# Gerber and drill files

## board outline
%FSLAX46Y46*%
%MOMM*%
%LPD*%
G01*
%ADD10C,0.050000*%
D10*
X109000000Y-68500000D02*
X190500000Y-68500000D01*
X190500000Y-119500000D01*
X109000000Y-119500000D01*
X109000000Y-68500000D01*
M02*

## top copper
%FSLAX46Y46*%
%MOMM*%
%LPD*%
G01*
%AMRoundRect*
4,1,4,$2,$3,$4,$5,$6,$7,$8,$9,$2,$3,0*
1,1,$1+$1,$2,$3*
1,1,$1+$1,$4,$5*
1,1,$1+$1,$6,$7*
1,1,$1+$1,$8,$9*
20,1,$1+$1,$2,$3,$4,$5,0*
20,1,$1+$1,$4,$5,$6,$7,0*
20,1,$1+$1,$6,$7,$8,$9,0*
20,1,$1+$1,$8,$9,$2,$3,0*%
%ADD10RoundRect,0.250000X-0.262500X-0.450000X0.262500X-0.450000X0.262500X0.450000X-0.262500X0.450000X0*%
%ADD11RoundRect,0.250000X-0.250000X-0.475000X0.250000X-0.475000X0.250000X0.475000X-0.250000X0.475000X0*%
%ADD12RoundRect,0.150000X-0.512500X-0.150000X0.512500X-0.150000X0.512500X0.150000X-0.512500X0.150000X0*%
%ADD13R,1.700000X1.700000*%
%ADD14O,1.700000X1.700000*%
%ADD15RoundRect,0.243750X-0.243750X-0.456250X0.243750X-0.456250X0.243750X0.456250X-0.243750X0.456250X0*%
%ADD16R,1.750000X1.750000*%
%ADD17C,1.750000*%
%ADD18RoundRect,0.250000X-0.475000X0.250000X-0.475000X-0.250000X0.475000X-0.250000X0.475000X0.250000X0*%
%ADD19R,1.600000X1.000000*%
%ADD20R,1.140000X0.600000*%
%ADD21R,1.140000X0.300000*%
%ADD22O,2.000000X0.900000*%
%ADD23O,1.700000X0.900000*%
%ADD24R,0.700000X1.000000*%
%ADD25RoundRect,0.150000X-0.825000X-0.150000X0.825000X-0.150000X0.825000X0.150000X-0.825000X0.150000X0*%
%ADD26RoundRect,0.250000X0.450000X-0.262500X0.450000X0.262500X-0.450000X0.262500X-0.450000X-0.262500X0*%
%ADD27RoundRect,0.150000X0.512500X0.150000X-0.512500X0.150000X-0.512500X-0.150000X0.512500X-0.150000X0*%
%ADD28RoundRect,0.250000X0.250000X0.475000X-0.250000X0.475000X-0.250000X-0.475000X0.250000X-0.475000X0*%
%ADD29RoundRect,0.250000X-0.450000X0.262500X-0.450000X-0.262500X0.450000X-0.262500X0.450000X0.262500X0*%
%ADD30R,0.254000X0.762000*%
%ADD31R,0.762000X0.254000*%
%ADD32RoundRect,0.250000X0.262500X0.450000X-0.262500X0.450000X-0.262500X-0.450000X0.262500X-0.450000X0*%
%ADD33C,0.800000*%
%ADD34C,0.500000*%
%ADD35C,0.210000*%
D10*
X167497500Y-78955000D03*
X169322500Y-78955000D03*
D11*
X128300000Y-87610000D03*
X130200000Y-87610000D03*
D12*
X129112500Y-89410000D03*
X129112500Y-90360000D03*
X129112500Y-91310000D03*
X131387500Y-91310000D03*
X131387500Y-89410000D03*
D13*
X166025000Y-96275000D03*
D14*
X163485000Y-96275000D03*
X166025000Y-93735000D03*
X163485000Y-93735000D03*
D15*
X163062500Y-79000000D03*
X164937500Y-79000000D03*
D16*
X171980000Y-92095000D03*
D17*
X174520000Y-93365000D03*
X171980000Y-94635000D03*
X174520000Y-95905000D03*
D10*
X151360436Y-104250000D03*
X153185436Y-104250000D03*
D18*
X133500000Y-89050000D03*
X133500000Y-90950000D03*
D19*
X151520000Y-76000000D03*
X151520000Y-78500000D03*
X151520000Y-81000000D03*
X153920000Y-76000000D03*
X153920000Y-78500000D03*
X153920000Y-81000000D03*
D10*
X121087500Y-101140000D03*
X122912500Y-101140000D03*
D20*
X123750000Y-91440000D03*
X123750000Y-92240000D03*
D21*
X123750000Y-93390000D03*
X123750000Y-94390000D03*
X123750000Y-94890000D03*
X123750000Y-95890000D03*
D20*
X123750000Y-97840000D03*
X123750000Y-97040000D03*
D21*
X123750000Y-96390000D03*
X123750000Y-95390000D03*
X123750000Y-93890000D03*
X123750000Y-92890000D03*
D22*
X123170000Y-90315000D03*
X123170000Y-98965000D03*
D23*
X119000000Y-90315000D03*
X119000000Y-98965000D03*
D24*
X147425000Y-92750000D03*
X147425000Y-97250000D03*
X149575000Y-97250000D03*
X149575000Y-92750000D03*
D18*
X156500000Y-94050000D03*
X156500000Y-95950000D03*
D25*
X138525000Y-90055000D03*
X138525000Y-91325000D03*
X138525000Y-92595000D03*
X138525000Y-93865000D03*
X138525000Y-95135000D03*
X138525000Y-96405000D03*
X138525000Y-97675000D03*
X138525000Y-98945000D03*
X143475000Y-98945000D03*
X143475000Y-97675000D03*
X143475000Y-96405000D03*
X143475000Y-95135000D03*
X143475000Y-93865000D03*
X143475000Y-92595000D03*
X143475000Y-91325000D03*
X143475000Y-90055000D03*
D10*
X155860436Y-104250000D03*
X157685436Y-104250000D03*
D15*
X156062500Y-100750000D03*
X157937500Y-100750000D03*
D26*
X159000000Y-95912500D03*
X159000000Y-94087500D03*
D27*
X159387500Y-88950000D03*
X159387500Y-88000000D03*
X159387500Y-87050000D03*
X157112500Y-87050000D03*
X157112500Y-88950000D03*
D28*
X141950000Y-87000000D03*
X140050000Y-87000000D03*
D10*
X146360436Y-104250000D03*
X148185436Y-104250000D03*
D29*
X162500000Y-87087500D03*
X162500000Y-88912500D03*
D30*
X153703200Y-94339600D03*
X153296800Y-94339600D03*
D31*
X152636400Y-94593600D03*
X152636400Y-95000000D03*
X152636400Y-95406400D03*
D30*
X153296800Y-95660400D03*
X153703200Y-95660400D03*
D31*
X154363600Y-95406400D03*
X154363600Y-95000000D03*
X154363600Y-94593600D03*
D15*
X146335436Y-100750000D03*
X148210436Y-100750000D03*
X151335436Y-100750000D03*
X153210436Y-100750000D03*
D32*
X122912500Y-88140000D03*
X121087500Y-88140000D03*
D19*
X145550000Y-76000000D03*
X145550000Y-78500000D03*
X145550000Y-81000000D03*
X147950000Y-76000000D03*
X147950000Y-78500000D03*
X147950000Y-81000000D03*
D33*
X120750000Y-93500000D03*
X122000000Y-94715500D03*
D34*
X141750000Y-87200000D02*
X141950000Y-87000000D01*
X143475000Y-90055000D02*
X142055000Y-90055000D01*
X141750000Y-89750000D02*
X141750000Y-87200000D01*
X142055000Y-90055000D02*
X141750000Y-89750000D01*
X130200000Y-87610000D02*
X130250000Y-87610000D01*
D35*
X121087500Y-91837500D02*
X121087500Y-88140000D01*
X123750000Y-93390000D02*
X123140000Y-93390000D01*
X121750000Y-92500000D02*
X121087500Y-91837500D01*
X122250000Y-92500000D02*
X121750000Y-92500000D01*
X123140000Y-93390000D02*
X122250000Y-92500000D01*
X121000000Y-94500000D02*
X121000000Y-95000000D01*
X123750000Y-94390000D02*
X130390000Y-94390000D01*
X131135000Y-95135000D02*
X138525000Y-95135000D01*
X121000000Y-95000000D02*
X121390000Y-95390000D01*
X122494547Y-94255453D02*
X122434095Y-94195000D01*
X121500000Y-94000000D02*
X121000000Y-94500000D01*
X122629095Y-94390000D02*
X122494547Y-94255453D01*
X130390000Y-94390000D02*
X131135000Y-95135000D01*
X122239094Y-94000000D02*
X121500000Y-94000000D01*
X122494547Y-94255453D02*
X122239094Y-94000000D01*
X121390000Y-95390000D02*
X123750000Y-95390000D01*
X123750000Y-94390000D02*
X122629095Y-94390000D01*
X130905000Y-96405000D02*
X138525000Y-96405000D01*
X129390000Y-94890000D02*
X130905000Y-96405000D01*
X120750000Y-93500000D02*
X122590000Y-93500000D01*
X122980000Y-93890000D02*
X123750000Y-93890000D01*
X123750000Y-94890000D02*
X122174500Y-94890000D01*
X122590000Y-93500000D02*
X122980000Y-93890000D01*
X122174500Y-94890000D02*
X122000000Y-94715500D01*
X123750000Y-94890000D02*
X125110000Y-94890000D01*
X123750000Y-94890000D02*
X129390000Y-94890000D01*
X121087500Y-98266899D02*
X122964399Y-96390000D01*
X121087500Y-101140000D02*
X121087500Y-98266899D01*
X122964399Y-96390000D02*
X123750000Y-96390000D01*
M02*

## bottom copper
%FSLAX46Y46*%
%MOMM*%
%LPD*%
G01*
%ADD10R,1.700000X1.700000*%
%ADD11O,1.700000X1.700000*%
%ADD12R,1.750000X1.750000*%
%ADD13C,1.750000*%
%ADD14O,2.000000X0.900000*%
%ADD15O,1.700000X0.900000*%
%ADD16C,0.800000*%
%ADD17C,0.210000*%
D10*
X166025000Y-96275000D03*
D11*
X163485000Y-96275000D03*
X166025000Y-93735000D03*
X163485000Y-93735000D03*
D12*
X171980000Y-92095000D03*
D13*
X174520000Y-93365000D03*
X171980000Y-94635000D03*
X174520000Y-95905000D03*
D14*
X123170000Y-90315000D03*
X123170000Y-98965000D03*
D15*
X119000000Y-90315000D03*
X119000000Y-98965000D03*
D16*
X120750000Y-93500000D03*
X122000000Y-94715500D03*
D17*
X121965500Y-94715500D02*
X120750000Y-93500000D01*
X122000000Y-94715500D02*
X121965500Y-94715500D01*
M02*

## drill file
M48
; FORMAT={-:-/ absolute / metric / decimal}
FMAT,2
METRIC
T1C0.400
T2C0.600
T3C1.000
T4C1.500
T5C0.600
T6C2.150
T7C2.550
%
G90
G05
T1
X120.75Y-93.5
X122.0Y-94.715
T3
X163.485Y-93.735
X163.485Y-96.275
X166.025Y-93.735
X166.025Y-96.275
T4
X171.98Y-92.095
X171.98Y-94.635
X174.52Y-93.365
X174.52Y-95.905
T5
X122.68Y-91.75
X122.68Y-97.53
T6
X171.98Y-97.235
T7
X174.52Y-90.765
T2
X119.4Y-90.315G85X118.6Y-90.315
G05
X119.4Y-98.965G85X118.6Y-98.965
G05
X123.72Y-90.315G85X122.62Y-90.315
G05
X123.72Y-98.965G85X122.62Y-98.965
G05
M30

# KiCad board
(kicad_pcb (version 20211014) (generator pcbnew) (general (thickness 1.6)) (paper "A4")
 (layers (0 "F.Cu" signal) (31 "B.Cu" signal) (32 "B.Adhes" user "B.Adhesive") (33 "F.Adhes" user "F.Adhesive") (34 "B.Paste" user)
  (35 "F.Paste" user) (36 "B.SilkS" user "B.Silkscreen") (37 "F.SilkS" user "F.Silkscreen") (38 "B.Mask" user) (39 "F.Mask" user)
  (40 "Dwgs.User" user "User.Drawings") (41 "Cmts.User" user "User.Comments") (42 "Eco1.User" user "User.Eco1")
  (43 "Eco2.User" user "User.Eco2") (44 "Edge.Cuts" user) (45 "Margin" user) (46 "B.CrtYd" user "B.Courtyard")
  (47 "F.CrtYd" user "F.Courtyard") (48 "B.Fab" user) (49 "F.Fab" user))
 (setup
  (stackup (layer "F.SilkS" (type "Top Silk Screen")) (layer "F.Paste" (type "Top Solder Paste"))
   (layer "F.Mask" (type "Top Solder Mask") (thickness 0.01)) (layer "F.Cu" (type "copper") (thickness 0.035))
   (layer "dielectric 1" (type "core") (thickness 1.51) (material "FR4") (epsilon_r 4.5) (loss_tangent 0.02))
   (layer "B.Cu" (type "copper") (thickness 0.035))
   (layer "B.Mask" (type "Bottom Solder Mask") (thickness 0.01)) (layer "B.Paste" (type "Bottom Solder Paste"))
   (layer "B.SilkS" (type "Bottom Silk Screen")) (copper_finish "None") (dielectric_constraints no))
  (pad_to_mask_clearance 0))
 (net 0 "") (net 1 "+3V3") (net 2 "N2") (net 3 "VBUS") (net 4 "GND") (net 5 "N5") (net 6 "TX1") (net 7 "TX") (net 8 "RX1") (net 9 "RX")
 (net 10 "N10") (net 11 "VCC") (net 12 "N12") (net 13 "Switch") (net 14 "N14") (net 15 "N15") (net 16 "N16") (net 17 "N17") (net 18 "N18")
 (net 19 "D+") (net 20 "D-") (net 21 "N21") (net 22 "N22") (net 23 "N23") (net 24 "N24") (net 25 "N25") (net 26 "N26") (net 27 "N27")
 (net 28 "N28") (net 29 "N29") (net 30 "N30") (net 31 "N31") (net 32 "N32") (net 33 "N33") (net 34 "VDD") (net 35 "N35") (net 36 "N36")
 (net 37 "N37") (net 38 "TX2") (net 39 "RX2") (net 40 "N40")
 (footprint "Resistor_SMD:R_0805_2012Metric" (layer "F.Cu") (at 168.41 78.955)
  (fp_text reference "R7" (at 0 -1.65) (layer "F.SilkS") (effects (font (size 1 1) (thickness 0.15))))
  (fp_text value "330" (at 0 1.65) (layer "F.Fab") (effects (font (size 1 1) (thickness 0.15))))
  (pad "1" smd roundrect (at -0.9125 0) (size 1.025 1.4) (layers "F.Cu" "F.Paste" "F.Mask") (roundrect_rratio 0.243902) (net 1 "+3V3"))
  (pad "2" smd roundrect (at 0.9125 0) (size 1.025 1.4) (layers "F.Cu" "F.Paste" "F.Mask") (roundrect_rratio 0.243902) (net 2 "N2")))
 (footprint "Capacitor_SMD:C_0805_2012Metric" (layer "F.Cu") (at 129.25 87.61)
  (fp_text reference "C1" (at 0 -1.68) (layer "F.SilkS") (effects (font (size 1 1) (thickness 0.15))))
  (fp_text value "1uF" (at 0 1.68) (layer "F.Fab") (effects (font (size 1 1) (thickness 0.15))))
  (pad "1" smd roundrect (at -0.95 0) (size 1 1.45) (layers "F.Cu" "F.Paste" "F.Mask") (roundrect_rratio 0.25) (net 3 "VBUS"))
  (pad "2" smd roundrect (at 0.95 0) (size 1 1.45) (layers "F.Cu" "F.Paste" "F.Mask") (roundrect_rratio 0.25) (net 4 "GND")))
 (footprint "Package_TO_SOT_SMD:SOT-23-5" (layer "F.Cu") (at 130.25 90.36)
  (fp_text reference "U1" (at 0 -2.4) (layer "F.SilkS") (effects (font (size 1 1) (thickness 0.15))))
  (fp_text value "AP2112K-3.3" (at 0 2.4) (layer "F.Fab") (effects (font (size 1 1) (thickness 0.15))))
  (pad "1" smd roundrect (at -1.1375 -0.95) (size 1.325 0.6) (layers "F.Cu" "F.Paste" "F.Mask") (roundrect_rratio 0.25) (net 3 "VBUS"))
  (pad "2" smd roundrect (at -1.1375 0) (size 1.325 0.6) (layers "F.Cu" "F.Paste" "F.Mask") (roundrect_rratio 0.25) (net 4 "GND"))
  (pad "3" smd roundrect (at -1.1375 0.95) (size 1.325 0.6) (layers "F.Cu" "F.Paste" "F.Mask") (roundrect_rratio 0.25) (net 3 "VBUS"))
  (pad "4" smd roundrect (at 1.1375 0.95) (size 1.325 0.6) (layers "F.Cu" "F.Paste" "F.Mask") (roundrect_rratio 0.25) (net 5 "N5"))
  (pad "5" smd roundrect (at 1.1375 -0.95) (size 1.325 0.6) (layers "F.Cu" "F.Paste" "F.Mask") (roundrect_rratio 0.25) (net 1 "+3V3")))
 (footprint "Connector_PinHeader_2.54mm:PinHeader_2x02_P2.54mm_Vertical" (layer "F.Cu") (at 166.025 96.275 180)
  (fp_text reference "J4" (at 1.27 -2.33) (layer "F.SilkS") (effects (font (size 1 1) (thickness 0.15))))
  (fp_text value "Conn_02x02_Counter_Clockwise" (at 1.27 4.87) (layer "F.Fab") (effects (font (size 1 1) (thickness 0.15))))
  (pad "1" thru_hole rect (at 0 0 180) (size 1.7 1.7) (drill 1) (layers *.Cu *.Mask) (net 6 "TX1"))
  (pad "2" thru_hole oval (at 2.54 0 180) (size 1.7 1.7) (drill 1) (layers *.Cu *.Mask) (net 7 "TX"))
  (pad "3" thru_hole oval (at 0 2.54 180) (size 1.7 1.7) (drill 1) (layers *.Cu *.Mask) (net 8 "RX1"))
  (pad "4" thru_hole oval (at 2.54 2.54 180) (size 1.7 1.7) (drill 1) (layers *.Cu *.Mask) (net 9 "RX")))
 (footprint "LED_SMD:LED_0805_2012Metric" (layer "F.Cu") (at 164 79)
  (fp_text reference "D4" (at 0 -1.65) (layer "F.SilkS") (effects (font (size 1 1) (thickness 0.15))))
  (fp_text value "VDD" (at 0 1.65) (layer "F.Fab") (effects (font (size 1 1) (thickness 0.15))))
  (pad "1" smd roundrect (at -0.9375 0) (size 0.975 1.4) (layers "F.Cu" "F.Paste" "F.Mask") (roundrect_rratio 0.25) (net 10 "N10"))
  (pad "2" smd roundrect (at 0.9375 0) (size 0.975 1.4) (layers "F.Cu" "F.Paste" "F.Mask") (roundrect_rratio 0.25) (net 2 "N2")))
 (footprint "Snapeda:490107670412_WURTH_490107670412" (layer "F.Cu") (at 173.25 94 90)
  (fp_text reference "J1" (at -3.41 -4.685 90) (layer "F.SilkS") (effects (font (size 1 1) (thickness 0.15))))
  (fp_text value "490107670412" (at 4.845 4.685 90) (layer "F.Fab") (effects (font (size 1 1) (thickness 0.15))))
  (pad "" np_thru_hole circle (at 3.235 1.27 90) (size 2.55 2.55) (drill 2.55) (layers *.Cu *.Mask))
  (pad "" np_thru_hole circle (at -3.235 -1.27 90) (size 2.15 2.15) (drill 2.15) (layers *.Cu *.Mask))
  (pad "1" thru_hole rect (at 1.905 -1.27 90) (size 1.75 1.75) (drill 1.5) (layers *.Cu *.Mask) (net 8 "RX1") (solder_mask_margin 0.102))
  (pad "2" thru_hole circle (at 0.635 1.27 90) (size 1.75 1.75) (drill 1.5) (layers *.Cu *.Mask) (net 4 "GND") (solder_mask_margin 0.102))
  (pad "3" thru_hole circle (at -0.635 -1.27 90) (size 1.75 1.75) (drill 1.5) (layers *.Cu *.Mask) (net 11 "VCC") (solder_mask_margin 0.102))
  (pad "4" thru_hole circle (at -1.905 1.27 90) (size 1.75 1.75) (drill 1.5) (layers *.Cu *.Mask) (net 6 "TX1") (solder_mask_margin 0.102)))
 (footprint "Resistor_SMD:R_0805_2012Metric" (layer "F.Cu") (at 152.272936 104.25)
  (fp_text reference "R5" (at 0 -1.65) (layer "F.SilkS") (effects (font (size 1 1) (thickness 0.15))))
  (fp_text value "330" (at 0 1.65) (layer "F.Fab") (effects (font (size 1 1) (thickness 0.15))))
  (pad "1" smd roundrect (at -0.9125 0) (size 1.025 1.4) (layers "F.Cu" "F.Paste" "F.Mask") (roundrect_rratio 0.243902) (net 1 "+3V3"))
  (pad "2" smd roundrect (at 0.9125 0) (size 1.025 1.4) (layers "F.Cu" "F.Paste" "F.Mask") (roundrect_rratio 0.243902) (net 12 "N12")))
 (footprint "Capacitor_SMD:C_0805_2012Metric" (layer "F.Cu") (at 133.5 90 -90)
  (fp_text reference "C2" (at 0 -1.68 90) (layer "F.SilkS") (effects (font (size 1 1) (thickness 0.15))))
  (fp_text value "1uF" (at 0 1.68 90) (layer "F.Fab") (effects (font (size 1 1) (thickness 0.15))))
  (pad "1" smd roundrect (at -0.95 0 270) (size 1 1.45) (layers "F.Cu" "F.Paste" "F.Mask") (roundrect_rratio 0.25) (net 1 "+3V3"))
  (pad "2" smd roundrect (at 0.95 0 270) (size 1 1.45) (layers "F.Cu" "F.Paste" "F.Mask") (roundrect_rratio 0.25) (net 4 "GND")))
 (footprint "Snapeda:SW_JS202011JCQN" (layer "F.Cu") (at 152.72 78.5)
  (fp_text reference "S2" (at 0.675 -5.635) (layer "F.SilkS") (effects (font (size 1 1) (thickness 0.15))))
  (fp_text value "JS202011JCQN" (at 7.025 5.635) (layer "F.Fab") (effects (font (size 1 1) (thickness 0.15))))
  (pad "1" smd rect (at -1.2 -2.5) (size 1.6 1) (layers "F.Cu" "F.Paste" "F.Mask") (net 1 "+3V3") (solder_mask_margin 0.102))
  (pad "2" smd rect (at -1.2 0) (size 1.6 1) (layers "F.Cu" "F.Paste" "F.Mask") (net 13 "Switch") (solder_mask_margin 0.102))
  (pad "3" smd rect (at -1.2 2.5) (size 1.6 1) (layers "F.Cu" "F.Paste" "F.Mask") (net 4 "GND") (solder_mask_margin 0.102))
  (pad "5" smd rect (at 1.2 -2.5) (size 1.6 1) (layers "F.Cu" "F.Paste" "F.Mask") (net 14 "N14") (solder_mask_margin 0.102))
  (pad "6" smd rect (at 1.2 0) (size 1.6 1) (layers "F.Cu" "F.Paste" "F.Mask") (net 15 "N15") (solder_mask_margin 0.102))
  (pad "7" smd rect (at 1.2 2.5) (size 1.6 1) (layers "F.Cu" "F.Paste" "F.Mask") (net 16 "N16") (solder_mask_margin 0.102)))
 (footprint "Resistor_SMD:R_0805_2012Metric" (layer "F.Cu") (at 122 101.14)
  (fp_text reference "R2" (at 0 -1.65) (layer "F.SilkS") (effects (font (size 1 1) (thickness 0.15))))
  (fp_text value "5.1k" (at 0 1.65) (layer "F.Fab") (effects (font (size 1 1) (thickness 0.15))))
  (pad "1" smd roundrect (at -0.9125 0) (size 1.025 1.4) (layers "F.Cu" "F.Paste" "F.Mask") (roundrect_rratio 0.243902) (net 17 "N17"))
  (pad "2" smd roundrect (at 0.9125 0) (size 1.025 1.4) (layers "F.Cu" "F.Paste" "F.Mask") (roundrect_rratio 0.243902) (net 4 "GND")))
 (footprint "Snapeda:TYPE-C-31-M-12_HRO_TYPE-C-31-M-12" (layer "F.Cu") (at 119 94.64 -90)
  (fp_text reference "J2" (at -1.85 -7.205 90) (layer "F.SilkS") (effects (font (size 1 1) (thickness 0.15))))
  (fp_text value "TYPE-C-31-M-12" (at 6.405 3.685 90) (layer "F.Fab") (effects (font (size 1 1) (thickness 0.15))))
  (pad "" np_thru_hole circle (at 2.89 -3.68 270) (size 0.6 0.6) (drill 0.6) (layers *.Cu *.Mask))
  (pad "" np_thru_hole circle (at -2.89 -3.68 270) (size 0.6 0.6) (drill 0.6) (layers *.Cu *.Mask))
  (pad "A1_B12" smd rect (at -3.2 -4.75 270) (size 0.6 1.14) (layers "F.Cu" "F.Paste") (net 4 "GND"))
  (pad "A4_B9" smd rect (at -2.4 -4.75 270) (size 0.6 1.14) (layers "F.Cu" "F.Paste") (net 3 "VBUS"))
  (pad "A5" smd rect (at -1.25 -4.75 270) (size 0.3 1.14) (layers "F.Cu" "F.Paste") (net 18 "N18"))
  (pad "A6" smd rect (at -0.25 -4.75 270) (size 0.3 1.14) (layers "F.Cu" "F.Paste") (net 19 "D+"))
  (pad "A7" smd rect (at 0.25 -4.75 270) (size 0.3 1.14) (layers "F.Cu" "F.Paste") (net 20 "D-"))
  (pad "A8" smd rect (at 1.25 -4.75 270) (size 0.3 1.14) (layers "F.Cu" "F.Paste") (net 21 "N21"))
  (pad "B1_A12" smd rect (at 3.2 -4.75 270) (size 0.6 1.14) (layers "F.Cu" "F.Paste") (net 4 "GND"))
  (pad "B4_A9" smd rect (at 2.4 -4.75 270) (size 0.6 1.14) (layers "F.Cu" "F.Paste") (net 3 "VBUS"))
  (pad "B5" smd rect (at 1.75 -4.75 270) (size 0.3 1.14) (layers "F.Cu" "F.Paste") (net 17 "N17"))
  (pad "B6" smd rect (at 0.75 -4.75 270) (size 0.3 1.14) (layers "F.Cu" "F.Paste") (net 19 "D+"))
  (pad "B7" smd rect (at -0.75 -4.75 270) (size 0.3 1.14) (layers "F.Cu" "F.Paste") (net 20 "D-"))
  (pad "B8" smd rect (at -1.75 -4.75 270) (size 0.3 1.14) (layers "F.Cu" "F.Paste") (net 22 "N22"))
  (pad "S1" thru_hole oval (at -4.325 -4.17 270) (size 0.9 2) (drill oval 0.6 1.7) (layers *.Cu *.Mask) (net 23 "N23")
   (solder_mask_margin 0.102))
  (pad "S2" thru_hole oval (at 4.325 -4.17 270) (size 0.9 2) (drill oval 0.6 1.7) (layers *.Cu *.Mask) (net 23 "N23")
   (solder_mask_margin 0.102))
  (pad "S3" thru_hole oval (at -4.325 0 270) (size 0.9 1.7) (drill oval 0.6 1.4) (layers *.Cu *.Mask) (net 23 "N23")
   (solder_mask_margin 0.102))
  (pad "S4" thru_hole oval (at 4.325 0 270) (size 0.9 1.7) (drill oval 0.6 1.4) (layers *.Cu *.Mask) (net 23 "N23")
   (solder_mask_margin 0.102)))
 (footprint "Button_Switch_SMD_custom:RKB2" (layer "F.Cu") (at 148.5 95 90)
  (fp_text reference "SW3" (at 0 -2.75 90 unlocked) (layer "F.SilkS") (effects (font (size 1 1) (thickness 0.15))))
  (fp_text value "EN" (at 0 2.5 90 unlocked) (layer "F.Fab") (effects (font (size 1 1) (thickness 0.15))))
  (pad "1" smd rect (at 2.25 -1.075 90) (size 1 0.7) (layers "F.Cu" "F.Paste" "F.Mask") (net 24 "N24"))
  (pad "1" smd rect (at -2.25 -1.075 90) (size 1 0.7) (layers "F.Cu" "F.Paste" "F.Mask") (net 24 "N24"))
  (pad "2" smd rect (at -2.25 1.075 90) (size 1 0.7) (layers "F.Cu" "F.Paste" "F.Mask") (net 4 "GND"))
  (pad "2" smd rect (at 2.25 1.075 90) (size 1 0.7) (layers "F.Cu" "F.Paste" "F.Mask") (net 4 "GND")))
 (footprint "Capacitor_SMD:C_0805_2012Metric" (layer "F.Cu") (at 156.5 95 -90)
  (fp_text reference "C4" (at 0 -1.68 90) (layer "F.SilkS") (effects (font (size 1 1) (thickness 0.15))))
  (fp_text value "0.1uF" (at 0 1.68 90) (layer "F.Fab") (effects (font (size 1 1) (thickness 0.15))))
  (pad "1" smd roundrect (at -0.95 0 270) (size 1 1.45) (layers "F.Cu" "F.Paste" "F.Mask") (roundrect_rratio 0.25) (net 1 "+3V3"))
  (pad "2" smd roundrect (at 0.95 0 270) (size 1 1.45) (layers "F.Cu" "F.Paste" "F.Mask") (roundrect_rratio 0.25) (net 4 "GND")))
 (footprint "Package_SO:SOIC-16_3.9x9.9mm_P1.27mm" (layer "F.Cu") (at 141 94.5)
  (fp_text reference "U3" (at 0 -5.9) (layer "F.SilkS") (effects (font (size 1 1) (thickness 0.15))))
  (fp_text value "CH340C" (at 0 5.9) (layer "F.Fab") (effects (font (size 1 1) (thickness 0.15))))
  (pad "1" smd roundrect (at -2.475 -4.445) (size 1.95 0.6) (layers "F.Cu" "F.Paste" "F.Mask") (roundrect_rratio 0.25) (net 4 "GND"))
  (pad "2" smd roundrect (at -2.475 -3.175) (size 1.95 0.6) (layers "F.Cu" "F.Paste" "F.Mask") (roundrect_rratio 0.25) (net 7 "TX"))
  (pad "3" smd roundrect (at -2.475 -1.905) (size 1.95 0.6) (layers "F.Cu" "F.Paste" "F.Mask") (roundrect_rratio 0.25) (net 9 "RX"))
  (pad "4" smd roundrect (at -2.475 -0.635) (size 1.95 0.6) (layers "F.Cu" "F.Paste" "F.Mask") (roundrect_rratio 0.25) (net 1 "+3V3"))
  (pad "5" smd roundrect (at -2.475 0.635) (size 1.95 0.6) (layers "F.Cu" "F.Paste" "F.Mask") (roundrect_rratio 0.25) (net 19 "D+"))
  (pad "6" smd roundrect (at -2.475 1.905) (size 1.95 0.6) (layers "F.Cu" "F.Paste" "F.Mask") (roundrect_rratio 0.25) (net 20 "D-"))
  (pad "7" smd roundrect (at -2.475 3.175) (size 1.95 0.6) (layers "F.Cu" "F.Paste" "F.Mask") (roundrect_rratio 0.25) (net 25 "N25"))
  (pad "8" smd roundrect (at -2.475 4.445) (size 1.95 0.6) (layers "F.Cu" "F.Paste" "F.Mask") (roundrect_rratio 0.25) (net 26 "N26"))
  (pad "9" smd roundrect (at 2.475 4.445) (size 1.95 0.6) (layers "F.Cu" "F.Paste" "F.Mask") (roundrect_rratio 0.25) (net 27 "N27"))
  (pad "10" smd roundrect (at 2.475 3.175) (size 1.95 0.6) (layers "F.Cu" "F.Paste" "F.Mask") (roundrect_rratio 0.25) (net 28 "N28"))
  (pad "11" smd roundrect (at 2.475 1.905) (size 1.95 0.6) (layers "F.Cu" "F.Paste" "F.Mask") (roundrect_rratio 0.25) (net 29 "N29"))
  (pad "12" smd roundrect (at 2.475 0.635) (size 1.95 0.6) (layers "F.Cu" "F.Paste" "F.Mask") (roundrect_rratio 0.25) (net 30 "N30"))
  (pad "13" smd roundrect (at 2.475 -0.635) (size 1.95 0.6) (layers "F.Cu" "F.Paste" "F.Mask") (roundrect_rratio 0.25) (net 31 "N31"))
  (pad "14" smd roundrect (at 2.475 -1.905) (size 1.95 0.6) (layers "F.Cu" "F.Paste" "F.Mask") (roundrect_rratio 0.25) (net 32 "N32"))
  (pad "15" smd roundrect (at 2.475 -3.175) (size 1.95 0.6) (layers "F.Cu" "F.Paste" "F.Mask") (roundrect_rratio 0.25) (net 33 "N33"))
  (pad "16" smd roundrect (at 2.475 -4.445) (size 1.95 0.6) (layers "F.Cu" "F.Paste" "F.Mask") (roundrect_rratio 0.25) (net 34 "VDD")))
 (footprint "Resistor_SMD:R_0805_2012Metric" (layer "F.Cu") (at 156.772936 104.25)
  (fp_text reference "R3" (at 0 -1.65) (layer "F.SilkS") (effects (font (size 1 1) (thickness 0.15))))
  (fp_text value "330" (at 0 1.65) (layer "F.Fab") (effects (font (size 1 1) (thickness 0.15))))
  (pad "1" smd roundrect (at -0.9125 0) (size 1.025 1.4) (layers "F.Cu" "F.Paste" "F.Mask") (roundrect_rratio 0.243902) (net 3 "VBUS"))
  (pad "2" smd roundrect (at 0.9125 0) (size 1.025 1.4) (layers "F.Cu" "F.Paste" "F.Mask") (roundrect_rratio 0.243902) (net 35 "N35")))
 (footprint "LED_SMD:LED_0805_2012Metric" (layer "F.Cu") (at 157 100.75)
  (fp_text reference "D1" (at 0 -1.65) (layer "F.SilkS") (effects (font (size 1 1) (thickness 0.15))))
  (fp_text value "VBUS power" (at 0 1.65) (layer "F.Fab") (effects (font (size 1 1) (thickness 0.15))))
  (pad "1" smd roundrect (at -0.9375 0) (size 0.975 1.4) (layers "F.Cu" "F.Paste" "F.Mask") (roundrect_rratio 0.25) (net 4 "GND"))
  (pad "2" smd roundrect (at 0.9375 0) (size 0.975 1.4) (layers "F.Cu" "F.Paste" "F.Mask") (roundrect_rratio 0.25) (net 35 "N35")))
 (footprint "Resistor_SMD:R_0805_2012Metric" (layer "F.Cu") (at 159 95 90)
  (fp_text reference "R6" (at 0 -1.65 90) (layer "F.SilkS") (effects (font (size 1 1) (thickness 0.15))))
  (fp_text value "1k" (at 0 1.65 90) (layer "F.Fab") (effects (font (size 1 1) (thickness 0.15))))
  (pad "1" smd roundrect (at -0.9125 0 90) (size 1.025 1.4) (layers "F.Cu" "F.Paste" "F.Mask") (roundrect_rratio 0.243902) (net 8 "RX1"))
  (pad "2" smd roundrect (at 0.9125 0 90) (size 1.025 1.4) (layers "F.Cu" "F.Paste" "F.Mask") (roundrect_rratio 0.243902) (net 6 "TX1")))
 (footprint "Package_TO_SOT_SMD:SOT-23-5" (layer "F.Cu") (at 158.25 88 180)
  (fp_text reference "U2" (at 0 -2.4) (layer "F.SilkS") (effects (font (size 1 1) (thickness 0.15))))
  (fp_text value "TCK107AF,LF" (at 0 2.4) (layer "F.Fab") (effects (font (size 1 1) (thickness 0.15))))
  (pad "1" smd roundrect (at -1.1375 -0.95 180) (size 1.325 0.6) (layers "F.Cu" "F.Paste" "F.Mask") (roundrect_rratio 0.25) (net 11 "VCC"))
  (pad "2" smd roundrect (at -1.1375 0 180) (size 1.325 0.6) (layers "F.Cu" "F.Paste" "F.Mask") (roundrect_rratio 0.25) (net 4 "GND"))
  (pad "3" smd roundrect (at -1.1375 0.95 180) (size 1.325 0.6) (layers "F.Cu" "F.Paste" "F.Mask") (roundrect_rratio 0.25) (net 24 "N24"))
  (pad "4" smd roundrect (at 1.1375 0.95 180) (size 1.325 0.6) (layers "F.Cu" "F.Paste" "F.Mask") (roundrect_rratio 0.25) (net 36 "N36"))
  (pad "5" smd roundrect (at 1.1375 -0.95 180) (size 1.325 0.6) (layers "F.Cu" "F.Paste" "F.Mask") (roundrect_rratio 0.25) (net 34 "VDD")))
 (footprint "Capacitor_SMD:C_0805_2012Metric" (layer "F.Cu") (at 141 87 180)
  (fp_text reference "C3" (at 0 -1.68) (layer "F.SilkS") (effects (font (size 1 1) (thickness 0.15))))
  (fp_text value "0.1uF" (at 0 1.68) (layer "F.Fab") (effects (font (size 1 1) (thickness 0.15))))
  (pad "1" smd roundrect (at -0.95 0 180) (size 1 1.45) (layers "F.Cu" "F.Paste" "F.Mask") (roundrect_rratio 0.25) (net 34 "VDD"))
  (pad "2" smd roundrect (at 0.95 0 180) (size 1 1.45) (layers "F.Cu" "F.Paste" "F.Mask") (roundrect_rratio 0.25) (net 4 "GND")))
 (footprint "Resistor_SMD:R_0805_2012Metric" (layer "F.Cu") (at 147.272936 104.25)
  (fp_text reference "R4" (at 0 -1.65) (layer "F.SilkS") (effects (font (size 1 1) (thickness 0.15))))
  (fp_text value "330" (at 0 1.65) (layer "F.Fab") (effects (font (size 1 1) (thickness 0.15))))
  (pad "1" smd roundrect (at -0.9125 0) (size 1.025 1.4) (layers "F.Cu" "F.Paste" "F.Mask") (roundrect_rratio 0.243902) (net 3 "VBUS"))
  (pad "2" smd roundrect (at 0.9125 0) (size 1.025 1.4) (layers "F.Cu" "F.Paste" "F.Mask") (roundrect_rratio 0.243902) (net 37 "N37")))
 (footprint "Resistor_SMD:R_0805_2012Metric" (layer "F.Cu") (at 162.5 88 -90)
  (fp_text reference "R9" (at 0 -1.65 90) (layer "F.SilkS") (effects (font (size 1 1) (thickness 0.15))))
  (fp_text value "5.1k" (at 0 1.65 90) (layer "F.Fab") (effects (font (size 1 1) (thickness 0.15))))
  (pad "1" smd roundrect (at -0.9125 0 270) (size 1.025 1.4) (layers "F.Cu" "F.Paste" "F.Mask") (roundrect_rratio 0.243902) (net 24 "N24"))
  (pad "2" smd roundrect (at 0.9125 0 270) (size 1.025 1.4) (layers "F.Cu" "F.Paste" "F.Mask") (roundrect_rratio 0.243902) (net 34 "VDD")))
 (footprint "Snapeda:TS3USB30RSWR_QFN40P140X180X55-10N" (layer "F.Cu") (at 153.5 95 -90)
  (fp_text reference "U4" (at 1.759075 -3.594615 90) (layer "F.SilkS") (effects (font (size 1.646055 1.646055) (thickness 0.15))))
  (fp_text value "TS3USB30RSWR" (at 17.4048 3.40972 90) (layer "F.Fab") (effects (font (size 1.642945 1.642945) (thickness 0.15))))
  (pad "1" smd rect (at -0.6604 -0.2032 180) (size 0.254 0.762) (layers "F.Cu" "F.Paste" "F.Mask") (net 6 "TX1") (solder_mask_margin 0.102))
  (pad "2" smd rect (at -0.6604 0.2032 180) (size 0.254 0.762) (layers "F.Cu" "F.Paste" "F.Mask") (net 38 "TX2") (solder_mask_margin 0.102))
  (pad "3" smd rect (at -0.4064 0.8636 90) (size 0.254 0.762) (layers "F.Cu" "F.Paste" "F.Mask") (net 7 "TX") (solder_mask_margin 0.102))
  (pad "4" smd rect (at 0 0.8636 90) (size 0.254 0.762) (layers "F.Cu" "F.Paste" "F.Mask") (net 4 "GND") (solder_mask_margin 0.102))
  (pad "5" smd rect (at 0.4064 0.8636 90) (size 0.254 0.762) (layers "F.Cu" "F.Paste" "F.Mask") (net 9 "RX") (solder_mask_margin 0.102))
  (pad "6" smd rect (at 0.6604 0.2032 180) (size 0.254 0.762) (layers "F.Cu" "F.Paste" "F.Mask") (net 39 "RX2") (solder_mask_margin 0.102))
  (pad "7" smd rect (at 0.6604 -0.2032 180) (size 0.254 0.762) (layers "F.Cu" "F.Paste" "F.Mask") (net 8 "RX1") (solder_mask_margin 0.102))
  (pad "8" smd rect (at 0.4064 -0.8636 90) (size 0.254 0.762) (layers "F.Cu" "F.Paste" "F.Mask") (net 4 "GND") (solder_mask_margin 0.102))
  (pad "9" smd rect (at 0 -0.8636 90) (size 0.254 0.762) (layers "F.Cu" "F.Paste" "F.Mask") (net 1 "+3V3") (solder_mask_margin 0.102))
  (pad "10" smd rect (at -0.4064 -0.8636 90) (size 0.254 0.762) (layers "F.Cu" "F.Paste" "F.Mask") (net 13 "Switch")
   (solder_mask_margin 0.102)))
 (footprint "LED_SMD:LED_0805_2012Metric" (layer "F.Cu") (at 147.272936 100.75)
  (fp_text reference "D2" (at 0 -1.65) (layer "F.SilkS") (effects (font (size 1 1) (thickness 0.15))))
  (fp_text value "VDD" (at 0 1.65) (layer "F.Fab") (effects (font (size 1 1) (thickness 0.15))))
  (pad "1" smd roundrect (at -0.9375 0) (size 0.975 1.4) (layers "F.Cu" "F.Paste" "F.Mask") (roundrect_rratio 0.25) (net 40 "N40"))
  (pad "2" smd roundrect (at 0.9375 0) (size 0.975 1.4) (layers "F.Cu" "F.Paste" "F.Mask") (roundrect_rratio 0.25) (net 37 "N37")))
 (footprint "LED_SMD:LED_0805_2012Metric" (layer "F.Cu") (at 152.272936 100.75)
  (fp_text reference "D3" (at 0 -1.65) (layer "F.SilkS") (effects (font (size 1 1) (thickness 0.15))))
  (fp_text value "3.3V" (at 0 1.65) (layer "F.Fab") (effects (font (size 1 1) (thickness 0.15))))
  (pad "1" smd roundrect (at -0.9375 0) (size 0.975 1.4) (layers "F.Cu" "F.Paste" "F.Mask") (roundrect_rratio 0.25) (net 4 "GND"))
  (pad "2" smd roundrect (at 0.9375 0) (size 0.975 1.4) (layers "F.Cu" "F.Paste" "F.Mask") (roundrect_rratio 0.25) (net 12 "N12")))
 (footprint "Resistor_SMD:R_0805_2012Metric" (layer "F.Cu") (at 122 88.14 180)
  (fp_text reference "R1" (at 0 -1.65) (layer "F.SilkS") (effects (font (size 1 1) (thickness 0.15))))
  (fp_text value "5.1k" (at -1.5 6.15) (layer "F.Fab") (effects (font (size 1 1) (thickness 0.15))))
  (pad "1" smd roundrect (at -0.9125 0 180) (size 1.025 1.4) (layers "F.Cu" "F.Paste" "F.Mask") (roundrect_rratio 0.243902) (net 4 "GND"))
  (pad "2" smd roundrect (at 0.9125 0 180) (size 1.025 1.4) (layers "F.Cu" "F.Paste" "F.Mask") (roundrect_rratio 0.243902) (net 18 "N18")))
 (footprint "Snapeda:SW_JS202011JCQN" (layer "F.Cu") (at 146.75 78.5)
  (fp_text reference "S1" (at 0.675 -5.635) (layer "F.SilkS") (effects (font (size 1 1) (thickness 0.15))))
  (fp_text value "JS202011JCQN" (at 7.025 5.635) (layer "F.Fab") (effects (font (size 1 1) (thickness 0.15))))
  (pad "1" smd rect (at -1.2 -2.5) (size 1.6 1) (layers "F.Cu" "F.Paste" "F.Mask") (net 3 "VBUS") (solder_mask_margin 0.102))
  (pad "2" smd rect (at -1.2 0) (size 1.6 1) (layers "F.Cu" "F.Paste" "F.Mask") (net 34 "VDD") (solder_mask_margin 0.102))
  (pad "3" smd rect (at -1.2 2.5) (size 1.6 1) (layers "F.Cu" "F.Paste" "F.Mask") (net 1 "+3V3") (solder_mask_margin 0.102))
  (pad "5" smd rect (at 1.2 -2.5) (size 1.6 1) (layers "F.Cu" "F.Paste" "F.Mask") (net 40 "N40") (solder_mask_margin 0.102))
  (pad "6" smd rect (at 1.2 0) (size 1.6 1) (layers "F.Cu" "F.Paste" "F.Mask") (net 4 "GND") (solder_mask_margin 0.102))
  (pad "7" smd rect (at 1.2 2.5) (size 1.6 1) (layers "F.Cu" "F.Paste" "F.Mask") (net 10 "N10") (solder_mask_margin 0.102)))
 (gr_rect (start 109 68.5) (end 190.5 119.5) (layer "Edge.Cuts") (width 0.05) (fill none))
 (segment (start 141.75 87.2) (end 141.95 87) (width 0.5) (layer "F.Cu") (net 34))
 (segment (start 143.475 90.055) (end 142.055 90.055) (width 0.5) (layer "F.Cu") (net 34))
 (segment (start 141.75 89.75) (end 141.75 87.2) (width 0.5) (layer "F.Cu") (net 34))
 (segment (start 142.055 90.055) (end 141.75 89.75) (width 0.5) (layer "F.Cu") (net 34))
 (segment (start 130.2 87.61) (end 130.25 87.61) (width 0.5) (layer "F.Cu") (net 4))
 (segment (start 121.0875 91.8375) (end 121.0875 88.14) (width 0.21) (layer "F.Cu") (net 18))
 (segment (start 123.75 93.39) (end 123.14 93.39) (width 0.21) (layer "F.Cu") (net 18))
 (segment (start 121.75 92.5) (end 121.0875 91.8375) (width 0.21) (layer "F.Cu") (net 18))
 (segment (start 122.25 92.5) (end 121.75 92.5) (width 0.21) (layer "F.Cu") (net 18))
 (segment (start 123.14 93.39) (end 122.25 92.5) (width 0.21) (layer "F.Cu") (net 18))
 (segment (start 121 94.5) (end 121 95) (width 0.21) (layer "F.Cu") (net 19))
 (segment (start 123.75 94.39) (end 130.39 94.39) (width 0.21) (layer "F.Cu") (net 19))
 (segment (start 131.135 95.135) (end 138.525 95.135) (width 0.21) (layer "F.Cu") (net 19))
 (segment (start 121 95) (end 121.39 95.39) (width 0.21) (layer "F.Cu") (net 19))
 (segment (start 122.494547 94.255453) (end 122.434095 94.195) (width 0.21) (layer "F.Cu") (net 19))
 (segment (start 121.5 94) (end 121 94.5) (width 0.21) (layer "F.Cu") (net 19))
 (segment (start 122.629095 94.39) (end 122.494547 94.255453) (width 0.21) (layer "F.Cu") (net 19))
 (segment (start 130.39 94.39) (end 131.135 95.135) (width 0.21) (layer "F.Cu") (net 19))
 (segment (start 122.239094 94) (end 121.5 94) (width 0.21) (layer "F.Cu") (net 19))
 (segment (start 122.494547 94.255453) (end 122.239094 94) (width 0.21) (layer "F.Cu") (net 19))
 (segment (start 121.39 95.39) (end 123.75 95.39) (width 0.21) (layer "F.Cu") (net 19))
 (segment (start 123.75 94.39) (end 122.629095 94.39) (width 0.21) (layer "F.Cu") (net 19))
 (segment (start 130.905 96.405) (end 138.525 96.405) (width 0.21) (layer "F.Cu") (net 20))
 (segment (start 129.39 94.89) (end 130.905 96.405) (width 0.21) (layer "F.Cu") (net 20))
 (segment (start 120.75 93.5) (end 122.59 93.5) (width 0.21) (layer "F.Cu") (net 20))
 (segment (start 122.98 93.89) (end 123.75 93.89) (width 0.21) (layer "F.Cu") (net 20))
 (segment (start 123.75 94.89) (end 122.1745 94.89) (width 0.21) (layer "F.Cu") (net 20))
 (segment (start 122.59 93.5) (end 122.98 93.89) (width 0.21) (layer "F.Cu") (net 20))
 (segment (start 122.1745 94.89) (end 122 94.7155) (width 0.21) (layer "F.Cu") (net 20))
 (segment (start 123.75 94.89) (end 125.11 94.89) (width 0.21) (layer "F.Cu") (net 20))
 (segment (start 123.75 94.89) (end 129.39 94.89) (width 0.21) (layer "F.Cu") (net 20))
 (via (at 120.75 93.5) (size 0.8) (drill 0.4) (layers "F.Cu" "B.Cu") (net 20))
 (via (at 122 94.7155) (size 0.8) (drill 0.4) (layers "F.Cu" "B.Cu") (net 20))
 (segment (start 121.9655 94.7155) (end 120.75 93.5) (width 0.21) (layer "B.Cu") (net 20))
 (segment (start 122 94.7155) (end 121.9655 94.7155) (width 0.21) (layer "B.Cu") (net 20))
 (segment (start 121.0875 98.266899) (end 122.964399 96.39) (width 0.21) (layer "F.Cu") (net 17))
 (segment (start 121.0875 101.14) (end 121.0875 98.266899) (width 0.21) (layer "F.Cu") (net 17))
 (segment (start 122.964399 96.39) (end 123.75 96.39) (width 0.21) (layer "F.Cu") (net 17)))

